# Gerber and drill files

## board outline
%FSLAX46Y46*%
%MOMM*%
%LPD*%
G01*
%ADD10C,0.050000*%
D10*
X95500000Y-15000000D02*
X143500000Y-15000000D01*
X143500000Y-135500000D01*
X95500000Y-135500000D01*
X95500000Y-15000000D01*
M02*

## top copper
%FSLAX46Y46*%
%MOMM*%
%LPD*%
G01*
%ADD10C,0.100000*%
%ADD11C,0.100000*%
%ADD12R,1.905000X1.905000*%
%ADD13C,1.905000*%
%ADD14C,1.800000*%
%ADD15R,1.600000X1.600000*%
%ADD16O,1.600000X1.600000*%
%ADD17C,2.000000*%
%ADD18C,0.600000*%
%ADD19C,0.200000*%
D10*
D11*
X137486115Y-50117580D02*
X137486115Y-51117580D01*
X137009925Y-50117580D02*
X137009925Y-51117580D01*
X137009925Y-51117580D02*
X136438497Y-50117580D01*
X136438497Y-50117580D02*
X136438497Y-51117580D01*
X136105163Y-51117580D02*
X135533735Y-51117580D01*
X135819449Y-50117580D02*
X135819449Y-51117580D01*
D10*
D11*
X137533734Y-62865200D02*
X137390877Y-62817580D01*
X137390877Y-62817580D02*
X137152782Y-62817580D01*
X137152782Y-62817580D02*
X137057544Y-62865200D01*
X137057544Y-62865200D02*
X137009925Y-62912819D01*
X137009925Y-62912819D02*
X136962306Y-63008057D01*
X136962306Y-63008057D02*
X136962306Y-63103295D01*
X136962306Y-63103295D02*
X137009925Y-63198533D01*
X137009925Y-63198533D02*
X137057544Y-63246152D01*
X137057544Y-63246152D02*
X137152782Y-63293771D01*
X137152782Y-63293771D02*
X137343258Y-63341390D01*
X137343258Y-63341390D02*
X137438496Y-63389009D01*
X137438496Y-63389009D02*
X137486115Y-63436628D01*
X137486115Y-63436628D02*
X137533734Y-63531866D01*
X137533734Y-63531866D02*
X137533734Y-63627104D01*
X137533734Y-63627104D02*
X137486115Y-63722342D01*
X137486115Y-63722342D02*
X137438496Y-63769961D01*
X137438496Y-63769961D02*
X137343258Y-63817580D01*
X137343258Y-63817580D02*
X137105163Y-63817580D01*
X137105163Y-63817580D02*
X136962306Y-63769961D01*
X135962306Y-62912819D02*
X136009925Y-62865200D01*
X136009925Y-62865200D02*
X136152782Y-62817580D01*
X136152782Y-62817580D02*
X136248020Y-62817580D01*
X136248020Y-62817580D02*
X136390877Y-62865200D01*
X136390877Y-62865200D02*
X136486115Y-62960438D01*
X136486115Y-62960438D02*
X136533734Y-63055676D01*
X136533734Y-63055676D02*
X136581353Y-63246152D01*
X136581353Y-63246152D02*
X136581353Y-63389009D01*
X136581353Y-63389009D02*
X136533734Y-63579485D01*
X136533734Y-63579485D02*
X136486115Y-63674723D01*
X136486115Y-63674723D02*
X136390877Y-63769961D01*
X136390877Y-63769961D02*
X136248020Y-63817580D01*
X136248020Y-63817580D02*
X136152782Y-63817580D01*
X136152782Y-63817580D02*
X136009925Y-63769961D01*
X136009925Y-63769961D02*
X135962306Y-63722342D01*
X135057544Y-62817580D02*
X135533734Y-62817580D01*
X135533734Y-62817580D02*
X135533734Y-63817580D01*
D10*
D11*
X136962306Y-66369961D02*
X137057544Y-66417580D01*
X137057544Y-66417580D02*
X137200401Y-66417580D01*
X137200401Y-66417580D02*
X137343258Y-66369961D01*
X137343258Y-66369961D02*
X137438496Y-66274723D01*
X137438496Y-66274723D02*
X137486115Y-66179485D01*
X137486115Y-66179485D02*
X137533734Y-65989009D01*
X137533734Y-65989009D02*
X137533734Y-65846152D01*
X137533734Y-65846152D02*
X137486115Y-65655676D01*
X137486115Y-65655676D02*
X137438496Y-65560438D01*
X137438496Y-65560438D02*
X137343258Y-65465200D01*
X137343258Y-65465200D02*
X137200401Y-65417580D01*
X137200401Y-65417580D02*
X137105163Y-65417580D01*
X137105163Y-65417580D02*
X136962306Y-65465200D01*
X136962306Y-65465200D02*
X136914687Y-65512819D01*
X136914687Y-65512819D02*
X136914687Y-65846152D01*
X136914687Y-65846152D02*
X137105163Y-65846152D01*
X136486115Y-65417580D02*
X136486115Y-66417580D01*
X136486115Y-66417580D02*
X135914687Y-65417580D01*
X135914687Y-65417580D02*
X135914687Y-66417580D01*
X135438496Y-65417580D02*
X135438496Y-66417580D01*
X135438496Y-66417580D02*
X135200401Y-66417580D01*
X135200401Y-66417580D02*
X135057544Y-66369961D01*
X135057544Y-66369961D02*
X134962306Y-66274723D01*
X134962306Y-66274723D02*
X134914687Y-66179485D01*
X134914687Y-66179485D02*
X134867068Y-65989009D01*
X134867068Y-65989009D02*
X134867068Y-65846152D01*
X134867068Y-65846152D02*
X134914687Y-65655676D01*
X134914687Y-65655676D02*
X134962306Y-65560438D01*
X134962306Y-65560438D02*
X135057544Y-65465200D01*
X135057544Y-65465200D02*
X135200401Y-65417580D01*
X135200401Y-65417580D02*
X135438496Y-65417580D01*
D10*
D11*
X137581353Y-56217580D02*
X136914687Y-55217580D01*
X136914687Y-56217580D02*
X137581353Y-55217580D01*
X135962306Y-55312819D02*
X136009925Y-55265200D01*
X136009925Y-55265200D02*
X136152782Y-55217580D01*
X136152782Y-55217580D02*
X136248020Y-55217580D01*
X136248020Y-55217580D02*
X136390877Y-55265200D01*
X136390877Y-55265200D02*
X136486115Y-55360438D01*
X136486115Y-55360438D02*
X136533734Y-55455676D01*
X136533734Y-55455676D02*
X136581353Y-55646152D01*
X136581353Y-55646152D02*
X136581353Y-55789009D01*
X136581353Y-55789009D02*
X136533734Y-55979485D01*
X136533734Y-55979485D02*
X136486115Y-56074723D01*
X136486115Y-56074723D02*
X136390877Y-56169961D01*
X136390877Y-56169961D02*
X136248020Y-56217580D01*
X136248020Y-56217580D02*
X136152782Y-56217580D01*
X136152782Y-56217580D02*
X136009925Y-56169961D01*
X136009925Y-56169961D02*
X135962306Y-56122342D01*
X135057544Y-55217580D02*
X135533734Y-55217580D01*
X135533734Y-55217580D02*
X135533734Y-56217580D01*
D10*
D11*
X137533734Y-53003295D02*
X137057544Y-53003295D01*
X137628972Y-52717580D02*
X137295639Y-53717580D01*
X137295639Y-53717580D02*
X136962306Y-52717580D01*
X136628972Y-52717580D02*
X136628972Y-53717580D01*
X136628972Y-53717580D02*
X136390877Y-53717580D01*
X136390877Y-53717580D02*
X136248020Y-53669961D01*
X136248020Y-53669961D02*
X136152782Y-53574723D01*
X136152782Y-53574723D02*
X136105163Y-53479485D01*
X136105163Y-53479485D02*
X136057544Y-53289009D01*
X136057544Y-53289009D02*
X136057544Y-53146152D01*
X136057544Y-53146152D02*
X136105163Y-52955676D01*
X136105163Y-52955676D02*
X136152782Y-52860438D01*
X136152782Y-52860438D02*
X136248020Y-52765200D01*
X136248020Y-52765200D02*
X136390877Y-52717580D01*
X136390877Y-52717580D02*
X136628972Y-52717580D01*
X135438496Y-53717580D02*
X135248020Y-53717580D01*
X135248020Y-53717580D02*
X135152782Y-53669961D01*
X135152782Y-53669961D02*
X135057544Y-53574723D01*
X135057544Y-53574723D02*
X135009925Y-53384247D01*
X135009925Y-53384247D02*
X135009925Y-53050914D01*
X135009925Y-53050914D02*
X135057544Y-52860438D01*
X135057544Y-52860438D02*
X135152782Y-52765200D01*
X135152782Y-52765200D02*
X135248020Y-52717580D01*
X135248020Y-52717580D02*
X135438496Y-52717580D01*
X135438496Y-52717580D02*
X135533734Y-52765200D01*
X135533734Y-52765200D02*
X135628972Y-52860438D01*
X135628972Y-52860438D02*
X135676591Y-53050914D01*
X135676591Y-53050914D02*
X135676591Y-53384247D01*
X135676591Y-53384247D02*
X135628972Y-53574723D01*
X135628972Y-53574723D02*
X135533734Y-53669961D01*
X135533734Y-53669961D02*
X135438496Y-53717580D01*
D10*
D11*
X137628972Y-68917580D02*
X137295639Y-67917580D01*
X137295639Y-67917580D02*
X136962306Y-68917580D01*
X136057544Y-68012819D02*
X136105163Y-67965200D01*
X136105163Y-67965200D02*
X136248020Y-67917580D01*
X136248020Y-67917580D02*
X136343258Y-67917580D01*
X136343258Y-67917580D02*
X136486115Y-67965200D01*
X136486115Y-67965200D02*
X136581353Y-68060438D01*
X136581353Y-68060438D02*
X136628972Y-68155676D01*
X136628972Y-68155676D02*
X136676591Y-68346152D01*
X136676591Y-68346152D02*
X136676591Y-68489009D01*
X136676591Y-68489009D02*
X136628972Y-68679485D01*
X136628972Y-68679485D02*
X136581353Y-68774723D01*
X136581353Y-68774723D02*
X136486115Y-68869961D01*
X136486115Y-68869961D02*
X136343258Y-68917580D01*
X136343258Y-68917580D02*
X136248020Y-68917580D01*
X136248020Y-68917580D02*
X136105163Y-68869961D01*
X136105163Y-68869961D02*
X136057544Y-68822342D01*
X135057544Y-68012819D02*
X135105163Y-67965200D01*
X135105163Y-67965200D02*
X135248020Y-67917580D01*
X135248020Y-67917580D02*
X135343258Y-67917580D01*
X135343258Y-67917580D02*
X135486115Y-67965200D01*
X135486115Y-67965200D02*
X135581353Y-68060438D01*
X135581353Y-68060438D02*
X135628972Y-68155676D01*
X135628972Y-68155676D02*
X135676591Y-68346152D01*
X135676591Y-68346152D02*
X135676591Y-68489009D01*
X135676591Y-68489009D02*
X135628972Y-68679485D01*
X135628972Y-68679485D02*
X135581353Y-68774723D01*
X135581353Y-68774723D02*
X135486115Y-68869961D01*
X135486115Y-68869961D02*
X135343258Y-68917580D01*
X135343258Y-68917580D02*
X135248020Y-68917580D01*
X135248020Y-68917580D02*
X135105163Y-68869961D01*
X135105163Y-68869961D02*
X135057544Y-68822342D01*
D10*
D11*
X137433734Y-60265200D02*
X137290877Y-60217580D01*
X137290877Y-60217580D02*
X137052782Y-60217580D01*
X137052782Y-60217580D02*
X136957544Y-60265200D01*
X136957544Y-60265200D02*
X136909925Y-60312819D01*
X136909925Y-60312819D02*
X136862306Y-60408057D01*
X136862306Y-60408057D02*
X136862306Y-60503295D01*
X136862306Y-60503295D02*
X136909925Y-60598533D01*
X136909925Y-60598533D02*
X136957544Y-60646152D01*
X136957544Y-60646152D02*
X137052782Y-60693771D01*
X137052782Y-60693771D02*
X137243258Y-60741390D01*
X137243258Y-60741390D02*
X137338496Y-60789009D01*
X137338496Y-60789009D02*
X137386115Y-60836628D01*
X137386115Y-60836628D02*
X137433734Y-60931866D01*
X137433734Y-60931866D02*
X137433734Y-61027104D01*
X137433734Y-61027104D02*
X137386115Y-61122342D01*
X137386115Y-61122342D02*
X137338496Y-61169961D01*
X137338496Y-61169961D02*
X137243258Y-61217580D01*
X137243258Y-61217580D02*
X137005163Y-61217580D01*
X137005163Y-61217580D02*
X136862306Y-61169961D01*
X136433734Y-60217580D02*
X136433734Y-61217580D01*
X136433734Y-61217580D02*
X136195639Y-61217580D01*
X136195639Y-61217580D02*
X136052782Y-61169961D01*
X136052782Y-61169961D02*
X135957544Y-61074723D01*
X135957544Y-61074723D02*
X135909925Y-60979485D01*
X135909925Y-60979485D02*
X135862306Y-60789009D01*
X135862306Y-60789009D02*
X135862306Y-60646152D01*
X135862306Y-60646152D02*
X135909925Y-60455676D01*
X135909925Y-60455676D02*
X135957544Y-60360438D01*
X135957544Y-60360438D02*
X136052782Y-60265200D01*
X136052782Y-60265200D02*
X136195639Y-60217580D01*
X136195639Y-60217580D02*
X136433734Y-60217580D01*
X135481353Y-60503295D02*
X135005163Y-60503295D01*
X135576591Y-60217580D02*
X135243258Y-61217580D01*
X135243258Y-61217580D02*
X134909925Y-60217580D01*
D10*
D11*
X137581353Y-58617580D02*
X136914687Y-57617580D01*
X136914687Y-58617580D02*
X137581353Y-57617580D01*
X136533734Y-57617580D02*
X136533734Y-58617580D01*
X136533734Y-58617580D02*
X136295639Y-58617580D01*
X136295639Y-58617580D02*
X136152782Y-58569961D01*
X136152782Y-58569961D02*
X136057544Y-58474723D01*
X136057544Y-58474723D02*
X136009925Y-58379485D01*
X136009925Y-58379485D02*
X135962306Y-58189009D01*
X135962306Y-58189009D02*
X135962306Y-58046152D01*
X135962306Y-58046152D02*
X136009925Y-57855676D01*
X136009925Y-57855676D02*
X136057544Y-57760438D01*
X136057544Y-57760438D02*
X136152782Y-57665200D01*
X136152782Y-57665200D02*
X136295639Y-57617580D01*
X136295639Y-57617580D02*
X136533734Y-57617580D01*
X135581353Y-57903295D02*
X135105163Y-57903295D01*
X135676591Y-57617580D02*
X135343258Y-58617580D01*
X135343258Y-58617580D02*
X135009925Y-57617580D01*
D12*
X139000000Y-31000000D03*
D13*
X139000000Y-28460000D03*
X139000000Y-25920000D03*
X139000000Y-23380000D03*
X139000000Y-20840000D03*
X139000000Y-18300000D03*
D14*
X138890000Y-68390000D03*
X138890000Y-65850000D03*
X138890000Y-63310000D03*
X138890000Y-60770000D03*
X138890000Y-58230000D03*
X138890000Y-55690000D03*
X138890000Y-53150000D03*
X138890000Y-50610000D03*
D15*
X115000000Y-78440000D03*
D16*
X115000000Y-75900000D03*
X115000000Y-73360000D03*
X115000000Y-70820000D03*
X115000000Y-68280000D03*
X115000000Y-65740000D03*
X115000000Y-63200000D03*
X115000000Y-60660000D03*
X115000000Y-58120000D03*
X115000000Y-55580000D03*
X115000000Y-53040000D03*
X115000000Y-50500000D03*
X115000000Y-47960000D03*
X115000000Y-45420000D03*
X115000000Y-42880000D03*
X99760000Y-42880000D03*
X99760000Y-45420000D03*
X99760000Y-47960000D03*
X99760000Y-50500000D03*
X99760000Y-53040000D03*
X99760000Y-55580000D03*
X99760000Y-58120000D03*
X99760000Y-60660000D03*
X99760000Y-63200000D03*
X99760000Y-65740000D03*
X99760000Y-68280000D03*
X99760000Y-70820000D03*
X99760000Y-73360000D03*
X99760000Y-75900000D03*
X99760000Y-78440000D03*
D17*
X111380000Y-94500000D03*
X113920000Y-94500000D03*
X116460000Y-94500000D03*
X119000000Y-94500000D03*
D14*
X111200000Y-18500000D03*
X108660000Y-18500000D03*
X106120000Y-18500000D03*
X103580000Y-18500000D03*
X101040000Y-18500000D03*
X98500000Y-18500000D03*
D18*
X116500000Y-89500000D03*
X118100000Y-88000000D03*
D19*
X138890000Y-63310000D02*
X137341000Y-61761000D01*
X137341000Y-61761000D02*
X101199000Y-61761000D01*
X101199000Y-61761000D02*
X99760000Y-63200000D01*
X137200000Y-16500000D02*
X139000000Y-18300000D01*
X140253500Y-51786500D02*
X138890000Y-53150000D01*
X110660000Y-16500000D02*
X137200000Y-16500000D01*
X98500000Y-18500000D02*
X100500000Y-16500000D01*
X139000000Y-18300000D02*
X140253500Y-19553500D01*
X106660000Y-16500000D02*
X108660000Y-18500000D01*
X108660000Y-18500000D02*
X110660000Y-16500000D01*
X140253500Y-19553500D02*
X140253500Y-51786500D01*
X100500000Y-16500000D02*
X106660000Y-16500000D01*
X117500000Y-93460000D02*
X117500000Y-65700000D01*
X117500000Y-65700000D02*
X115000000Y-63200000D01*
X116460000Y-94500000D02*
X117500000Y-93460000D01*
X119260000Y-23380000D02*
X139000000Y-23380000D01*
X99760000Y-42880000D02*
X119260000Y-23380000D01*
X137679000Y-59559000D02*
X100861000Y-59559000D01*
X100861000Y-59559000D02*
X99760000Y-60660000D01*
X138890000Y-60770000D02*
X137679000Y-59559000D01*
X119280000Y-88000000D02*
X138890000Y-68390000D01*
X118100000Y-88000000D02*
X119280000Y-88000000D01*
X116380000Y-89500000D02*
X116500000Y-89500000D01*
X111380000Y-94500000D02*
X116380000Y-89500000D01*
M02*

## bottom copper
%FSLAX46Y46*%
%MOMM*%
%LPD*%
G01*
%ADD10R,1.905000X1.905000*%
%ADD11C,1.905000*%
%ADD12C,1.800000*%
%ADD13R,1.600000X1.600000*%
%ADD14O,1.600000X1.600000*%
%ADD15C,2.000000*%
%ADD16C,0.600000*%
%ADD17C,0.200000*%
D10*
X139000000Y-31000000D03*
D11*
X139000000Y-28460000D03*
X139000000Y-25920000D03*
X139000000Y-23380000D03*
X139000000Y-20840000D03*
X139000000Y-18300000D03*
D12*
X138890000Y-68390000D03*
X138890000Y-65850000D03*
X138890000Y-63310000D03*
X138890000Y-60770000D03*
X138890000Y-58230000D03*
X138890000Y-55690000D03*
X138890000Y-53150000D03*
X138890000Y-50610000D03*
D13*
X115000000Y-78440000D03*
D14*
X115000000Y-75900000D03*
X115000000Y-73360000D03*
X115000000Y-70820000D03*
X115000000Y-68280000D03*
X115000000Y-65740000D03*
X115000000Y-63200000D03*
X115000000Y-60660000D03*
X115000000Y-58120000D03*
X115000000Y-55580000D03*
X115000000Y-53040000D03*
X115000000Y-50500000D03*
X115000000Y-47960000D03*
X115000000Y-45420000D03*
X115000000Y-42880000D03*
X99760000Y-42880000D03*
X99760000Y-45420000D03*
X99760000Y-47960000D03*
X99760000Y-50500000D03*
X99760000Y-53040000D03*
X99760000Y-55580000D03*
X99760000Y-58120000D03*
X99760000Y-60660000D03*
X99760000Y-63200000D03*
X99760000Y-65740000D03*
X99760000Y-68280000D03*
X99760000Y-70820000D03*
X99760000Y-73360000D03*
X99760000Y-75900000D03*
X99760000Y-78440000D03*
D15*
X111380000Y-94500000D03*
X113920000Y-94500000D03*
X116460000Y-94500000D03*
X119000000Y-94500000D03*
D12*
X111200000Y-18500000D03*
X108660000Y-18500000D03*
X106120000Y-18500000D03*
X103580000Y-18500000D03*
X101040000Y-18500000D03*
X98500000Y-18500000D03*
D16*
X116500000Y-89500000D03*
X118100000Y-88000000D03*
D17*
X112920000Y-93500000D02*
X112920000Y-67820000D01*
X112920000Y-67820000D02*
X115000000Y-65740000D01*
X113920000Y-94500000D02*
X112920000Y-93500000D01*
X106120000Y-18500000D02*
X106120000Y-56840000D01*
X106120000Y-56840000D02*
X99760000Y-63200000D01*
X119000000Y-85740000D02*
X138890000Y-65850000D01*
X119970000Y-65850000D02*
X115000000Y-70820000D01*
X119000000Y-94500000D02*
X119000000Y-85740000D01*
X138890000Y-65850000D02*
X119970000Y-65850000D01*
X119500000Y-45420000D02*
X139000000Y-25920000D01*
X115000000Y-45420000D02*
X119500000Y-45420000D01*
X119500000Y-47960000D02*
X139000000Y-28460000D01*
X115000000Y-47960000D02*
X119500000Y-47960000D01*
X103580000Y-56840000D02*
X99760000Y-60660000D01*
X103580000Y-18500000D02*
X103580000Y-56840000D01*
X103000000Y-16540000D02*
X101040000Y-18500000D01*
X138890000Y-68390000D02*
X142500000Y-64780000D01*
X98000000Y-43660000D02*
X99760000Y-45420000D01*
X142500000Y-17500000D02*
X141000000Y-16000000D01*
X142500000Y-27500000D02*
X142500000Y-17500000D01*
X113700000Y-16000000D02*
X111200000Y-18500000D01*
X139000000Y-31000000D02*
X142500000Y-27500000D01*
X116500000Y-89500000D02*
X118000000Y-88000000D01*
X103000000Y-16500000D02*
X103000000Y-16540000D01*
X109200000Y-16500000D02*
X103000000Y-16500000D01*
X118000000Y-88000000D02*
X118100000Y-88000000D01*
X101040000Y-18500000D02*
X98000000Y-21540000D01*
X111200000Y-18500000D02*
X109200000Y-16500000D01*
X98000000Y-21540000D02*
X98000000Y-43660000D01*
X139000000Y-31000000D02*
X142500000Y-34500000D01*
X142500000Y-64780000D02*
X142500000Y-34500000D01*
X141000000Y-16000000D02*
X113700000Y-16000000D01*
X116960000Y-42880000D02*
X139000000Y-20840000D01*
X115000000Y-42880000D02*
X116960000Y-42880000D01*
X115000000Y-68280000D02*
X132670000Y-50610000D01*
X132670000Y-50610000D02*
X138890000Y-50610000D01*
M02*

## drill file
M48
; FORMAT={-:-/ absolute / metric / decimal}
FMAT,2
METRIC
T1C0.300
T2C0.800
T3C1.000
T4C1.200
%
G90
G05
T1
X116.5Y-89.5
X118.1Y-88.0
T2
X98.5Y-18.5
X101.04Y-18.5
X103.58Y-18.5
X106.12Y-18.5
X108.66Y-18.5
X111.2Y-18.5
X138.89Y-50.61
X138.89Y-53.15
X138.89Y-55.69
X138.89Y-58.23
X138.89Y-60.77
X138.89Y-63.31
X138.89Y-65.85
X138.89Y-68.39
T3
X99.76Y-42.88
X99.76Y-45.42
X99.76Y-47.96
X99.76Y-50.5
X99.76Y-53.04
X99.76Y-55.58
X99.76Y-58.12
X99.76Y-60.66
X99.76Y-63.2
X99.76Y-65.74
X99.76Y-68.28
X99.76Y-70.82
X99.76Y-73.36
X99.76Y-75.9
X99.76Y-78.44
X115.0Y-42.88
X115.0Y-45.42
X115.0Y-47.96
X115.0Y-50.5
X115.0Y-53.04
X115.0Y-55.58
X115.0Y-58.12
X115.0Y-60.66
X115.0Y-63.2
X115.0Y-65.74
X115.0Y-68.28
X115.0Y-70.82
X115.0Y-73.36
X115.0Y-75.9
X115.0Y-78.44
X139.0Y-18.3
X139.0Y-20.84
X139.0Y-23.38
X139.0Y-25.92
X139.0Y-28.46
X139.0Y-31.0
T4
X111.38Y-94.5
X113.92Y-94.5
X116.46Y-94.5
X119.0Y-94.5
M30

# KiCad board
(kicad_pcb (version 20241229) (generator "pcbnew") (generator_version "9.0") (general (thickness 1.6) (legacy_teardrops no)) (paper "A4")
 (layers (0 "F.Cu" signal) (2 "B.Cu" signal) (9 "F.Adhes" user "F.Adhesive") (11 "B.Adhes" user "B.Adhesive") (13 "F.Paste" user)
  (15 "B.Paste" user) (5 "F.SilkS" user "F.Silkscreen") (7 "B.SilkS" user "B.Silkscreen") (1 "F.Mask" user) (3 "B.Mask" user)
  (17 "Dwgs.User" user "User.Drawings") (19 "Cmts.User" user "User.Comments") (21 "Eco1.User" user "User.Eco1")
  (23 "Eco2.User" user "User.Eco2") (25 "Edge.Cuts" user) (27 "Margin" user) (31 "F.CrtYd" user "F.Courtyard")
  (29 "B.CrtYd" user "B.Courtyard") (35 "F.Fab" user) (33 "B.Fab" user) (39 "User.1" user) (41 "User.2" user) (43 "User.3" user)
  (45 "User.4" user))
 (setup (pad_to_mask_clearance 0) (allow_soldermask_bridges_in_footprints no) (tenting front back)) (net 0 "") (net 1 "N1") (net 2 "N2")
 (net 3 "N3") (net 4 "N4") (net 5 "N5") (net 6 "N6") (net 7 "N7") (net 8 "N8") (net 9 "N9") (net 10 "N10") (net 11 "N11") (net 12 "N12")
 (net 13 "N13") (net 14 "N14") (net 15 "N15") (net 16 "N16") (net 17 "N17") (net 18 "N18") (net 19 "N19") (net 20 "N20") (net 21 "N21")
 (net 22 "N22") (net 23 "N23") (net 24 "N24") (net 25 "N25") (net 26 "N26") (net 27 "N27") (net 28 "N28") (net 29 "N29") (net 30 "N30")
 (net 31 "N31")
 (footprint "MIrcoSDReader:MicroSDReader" (layer "F.Cu") (at 139 31 180)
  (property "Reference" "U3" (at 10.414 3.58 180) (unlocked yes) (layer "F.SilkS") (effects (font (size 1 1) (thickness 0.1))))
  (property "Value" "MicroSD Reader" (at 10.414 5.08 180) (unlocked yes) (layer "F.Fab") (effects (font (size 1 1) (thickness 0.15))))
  (pad "1" thru_hole rect (at 0 0 180) (size 1.905 1.905) (drill 1) (layers "*.Cu" "*.Mask") (remove_unused_layers no) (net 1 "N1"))
  (pad "2" thru_hole circle (at 0 2.54 180) (size 1.905 1.905) (drill 1) (layers "*.Cu" "*.Mask") (remove_unused_layers no) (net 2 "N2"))
  (pad "3" thru_hole circle (at 0 5.08 180) (size 1.905 1.905) (drill 1) (layers "*.Cu" "*.Mask") (remove_unused_layers no) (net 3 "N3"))
  (pad "4" thru_hole circle (at 0 7.62 180) (size 1.905 1.905) (drill 1) (layers "*.Cu" "*.Mask") (remove_unused_layers no) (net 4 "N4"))
  (pad "5" thru_hole circle (at 0 10.16 180) (size 1.905 1.905) (drill 1) (layers "*.Cu" "*.Mask") (remove_unused_layers no) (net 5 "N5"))
  (pad "6" thru_hole circle (at 0 12.7 180) (size 1.905 1.905) (drill 1) (layers "*.Cu" "*.Mask") (remove_unused_layers no) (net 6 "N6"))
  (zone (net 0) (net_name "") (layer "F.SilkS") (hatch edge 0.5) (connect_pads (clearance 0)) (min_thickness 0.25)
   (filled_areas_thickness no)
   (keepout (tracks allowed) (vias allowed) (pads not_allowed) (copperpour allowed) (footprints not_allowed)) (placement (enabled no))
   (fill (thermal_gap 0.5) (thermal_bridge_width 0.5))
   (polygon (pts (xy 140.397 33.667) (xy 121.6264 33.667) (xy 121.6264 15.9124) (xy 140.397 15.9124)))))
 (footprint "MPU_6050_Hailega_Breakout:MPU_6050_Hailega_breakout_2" (layer "F.Cu") (at 138.89 68.39 180)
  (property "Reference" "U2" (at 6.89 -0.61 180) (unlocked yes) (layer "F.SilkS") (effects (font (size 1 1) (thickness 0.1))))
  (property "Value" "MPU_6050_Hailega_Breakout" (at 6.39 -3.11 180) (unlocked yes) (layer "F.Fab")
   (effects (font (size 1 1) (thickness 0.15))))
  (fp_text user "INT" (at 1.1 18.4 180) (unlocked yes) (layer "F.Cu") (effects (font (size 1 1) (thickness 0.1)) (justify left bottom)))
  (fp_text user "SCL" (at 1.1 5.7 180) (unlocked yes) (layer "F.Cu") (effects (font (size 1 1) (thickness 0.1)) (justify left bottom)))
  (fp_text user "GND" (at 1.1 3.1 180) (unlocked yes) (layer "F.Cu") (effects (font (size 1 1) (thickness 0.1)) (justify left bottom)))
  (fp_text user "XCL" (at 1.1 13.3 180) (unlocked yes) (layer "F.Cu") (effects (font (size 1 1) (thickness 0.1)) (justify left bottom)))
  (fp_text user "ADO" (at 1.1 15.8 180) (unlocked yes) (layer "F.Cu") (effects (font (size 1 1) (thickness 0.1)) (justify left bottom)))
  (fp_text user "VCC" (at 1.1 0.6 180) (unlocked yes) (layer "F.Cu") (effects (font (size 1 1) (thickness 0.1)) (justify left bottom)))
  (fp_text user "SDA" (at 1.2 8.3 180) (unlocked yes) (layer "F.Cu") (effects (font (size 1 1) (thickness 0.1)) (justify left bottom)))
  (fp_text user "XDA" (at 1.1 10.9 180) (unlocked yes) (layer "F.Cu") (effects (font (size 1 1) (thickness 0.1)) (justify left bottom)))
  (pad "1" thru_hole circle (at 0 0 180) (size 1.8 1.8) (drill 0.8) (layers "*.Cu" "*.Mask") (remove_unused_layers no) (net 1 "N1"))
  (pad "2" thru_hole circle (at 0 2.54 180) (size 1.8 1.8) (drill 0.8) (layers "*.Cu" "*.Mask") (remove_unused_layers no) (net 6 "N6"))
  (pad "3" thru_hole circle (at 0 5.08 180) (size 1.8 1.8) (drill 0.8) (layers "*.Cu" "*.Mask") (remove_unused_layers no) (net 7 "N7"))
  (pad "4" thru_hole circle (at 0 7.62 180) (size 1.8 1.8) (drill 0.8) (layers "*.Cu" "*.Mask") (remove_unused_layers no) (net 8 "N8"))
  (pad "5" thru_hole circle (at 0 10.16 180) (size 1.8 1.8) (drill 0.8) (layers "*.Cu" "*.Mask") (remove_unused_layers no) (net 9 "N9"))
  (pad "6" thru_hole circle (at 0 12.7 180) (size 1.8 1.8) (drill 0.8) (layers "*.Cu" "*.Mask") (remove_unused_layers no) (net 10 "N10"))
  (pad "7" thru_hole circle (at 0 15.24 180) (size 1.8 1.8) (drill 0.8) (layers "*.Cu" "*.Mask") (remove_unused_layers no) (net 6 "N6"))
  (pad "8" thru_hole circle (at 0 17.78 180) (size 1.8 1.8) (drill 0.8) (layers "*.Cu" "*.Mask") (remove_unused_layers no) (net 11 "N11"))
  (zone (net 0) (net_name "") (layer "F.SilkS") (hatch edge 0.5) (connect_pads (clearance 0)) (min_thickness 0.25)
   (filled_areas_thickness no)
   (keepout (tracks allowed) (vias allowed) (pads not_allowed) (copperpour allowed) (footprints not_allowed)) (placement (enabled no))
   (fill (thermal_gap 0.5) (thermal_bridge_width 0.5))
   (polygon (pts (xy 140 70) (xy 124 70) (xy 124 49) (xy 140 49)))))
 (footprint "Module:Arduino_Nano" (layer "F.Cu") (at 115 78.44 180)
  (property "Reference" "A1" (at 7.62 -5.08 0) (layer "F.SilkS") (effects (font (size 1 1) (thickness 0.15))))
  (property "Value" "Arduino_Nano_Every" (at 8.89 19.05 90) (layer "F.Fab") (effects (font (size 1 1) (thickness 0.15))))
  (pad "1" thru_hole rect (at 0 0 180) (size 1.6 1.6) (drill 1) (layers "*.Cu" "*.Mask") (remove_unused_layers no) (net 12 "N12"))
  (pad "2" thru_hole oval (at 0 2.54 180) (size 1.6 1.6) (drill 1) (layers "*.Cu" "*.Mask") (remove_unused_layers no) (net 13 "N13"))
  (pad "3" thru_hole oval (at 0 5.08 180) (size 1.6 1.6) (drill 1) (layers "*.Cu" "*.Mask") (remove_unused_layers no) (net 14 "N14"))
  (pad "4" thru_hole oval (at 0 7.62 180) (size 1.6 1.6) (drill 1) (layers "*.Cu" "*.Mask") (remove_unused_layers no) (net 6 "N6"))
  (pad "5" thru_hole oval (at 0 10.16 180) (size 1.6 1.6) (drill 1) (layers "*.Cu" "*.Mask") (remove_unused_layers no) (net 11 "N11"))
  (pad "6" thru_hole oval (at 0 12.7 180) (size 1.6 1.6) (drill 1) (layers "*.Cu" "*.Mask") (remove_unused_layers no) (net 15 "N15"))
  (pad "7" thru_hole oval (at 0 15.24 180) (size 1.6 1.6) (drill 1) (layers "*.Cu" "*.Mask") (remove_unused_layers no) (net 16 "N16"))
  (pad "8" thru_hole oval (at 0 17.78 180) (size 1.6 1.6) (drill 1) (layers "*.Cu" "*.Mask") (remove_unused_layers no) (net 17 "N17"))
  (pad "9" thru_hole oval (at 0 20.32 180) (size 1.6 1.6) (drill 1) (layers "*.Cu" "*.Mask") (remove_unused_layers no) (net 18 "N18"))
  (pad "10" thru_hole oval (at 0 22.86 180) (size 1.6 1.6) (drill 1) (layers "*.Cu" "*.Mask") (remove_unused_layers no) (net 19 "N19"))
  (pad "11" thru_hole oval (at 0 25.4 180) (size 1.6 1.6) (drill 1) (layers "*.Cu" "*.Mask") (remove_unused_layers no) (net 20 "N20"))
  (pad "12" thru_hole oval (at 0 27.94 180) (size 1.6 1.6) (drill 1) (layers "*.Cu" "*.Mask") (remove_unused_layers no) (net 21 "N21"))
  (pad "13" thru_hole oval (at 0 30.48 180) (size 1.6 1.6) (drill 1) (layers "*.Cu" "*.Mask") (remove_unused_layers no) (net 2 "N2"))
  (pad "14" thru_hole oval (at 0 33.02 180) (size 1.6 1.6) (drill 1) (layers "*.Cu" "*.Mask") (remove_unused_layers no) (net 3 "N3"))
  (pad "15" thru_hole oval (at 0 35.56 180) (size 1.6 1.6) (drill 1) (layers "*.Cu" "*.Mask") (remove_unused_layers no) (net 5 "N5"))
  (pad "16" thru_hole oval (at 15.24 35.56 180) (size 1.6 1.6) (drill 1) (layers "*.Cu" "*.Mask") (remove_unused_layers no) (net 4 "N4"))
  (pad "17" thru_hole oval (at 15.24 33.02 180) (size 1.6 1.6) (drill 1) (layers "*.Cu" "*.Mask") (remove_unused_layers no) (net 1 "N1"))
  (pad "18" thru_hole oval (at 15.24 30.48 180) (size 1.6 1.6) (drill 1) (layers "*.Cu" "*.Mask") (remove_unused_layers no) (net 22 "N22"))
  (pad "19" thru_hole oval (at 15.24 27.94 180) (size 1.6 1.6) (drill 1) (layers "*.Cu" "*.Mask") (remove_unused_layers no) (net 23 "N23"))
  (pad "20" thru_hole oval (at 15.24 25.4 180) (size 1.6 1.6) (drill 1) (layers "*.Cu" "*.Mask") (remove_unused_layers no) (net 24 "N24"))
  (pad "21" thru_hole oval (at 15.24 22.86 180) (size 1.6 1.6) (drill 1) (layers "*.Cu" "*.Mask") (remove_unused_layers no) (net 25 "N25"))
  (pad "22" thru_hole oval (at 15.24 20.32 180) (size 1.6 1.6) (drill 1) (layers "*.Cu" "*.Mask") (remove_unused_layers no) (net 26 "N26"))
  (pad "23" thru_hole oval (at 15.24 17.78 180) (size 1.6 1.6) (drill 1) (layers "*.Cu" "*.Mask") (remove_unused_layers no) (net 8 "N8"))
  (pad "24" thru_hole oval (at 15.24 15.24 180) (size 1.6 1.6) (drill 1) (layers "*.Cu" "*.Mask") (remove_unused_layers no) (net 7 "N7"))
  (pad "25" thru_hole oval (at 15.24 12.7 180) (size 1.6 1.6) (drill 1) (layers "*.Cu" "*.Mask") (remove_unused_layers no) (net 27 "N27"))
  (pad "26" thru_hole oval (at 15.24 10.16 180) (size 1.6 1.6) (drill 1) (layers "*.Cu" "*.Mask") (remove_unused_layers no) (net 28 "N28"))
  (pad "27" thru_hole oval (at 15.24 7.62 180) (size 1.6 1.6) (drill 1) (layers "*.Cu" "*.Mask") (remove_unused_layers no) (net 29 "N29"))
  (pad "28" thru_hole oval (at 15.24 5.08 180) (size 1.6 1.6) (drill 1) (layers "*.Cu" "*.Mask") (remove_unused_layers no) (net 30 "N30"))
  (pad "29" thru_hole oval (at 15.24 2.54 180) (size 1.6 1.6) (drill 1) (layers "*.Cu" "*.Mask") (remove_unused_layers no) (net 6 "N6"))
  (pad "30" thru_hole oval (at 15.24 0 180) (size 1.6 1.6) (drill 1) (layers "*.Cu" "*.Mask") (remove_unused_layers no) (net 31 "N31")))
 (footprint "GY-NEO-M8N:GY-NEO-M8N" (layer "F.Cu") (at 111.38 94.5)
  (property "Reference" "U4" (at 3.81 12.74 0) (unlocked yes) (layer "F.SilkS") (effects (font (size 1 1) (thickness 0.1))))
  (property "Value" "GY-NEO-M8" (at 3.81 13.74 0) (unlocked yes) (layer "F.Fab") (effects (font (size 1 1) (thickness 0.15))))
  (pad "1" thru_hole circle (at 0 0) (size 2 2) (drill 1.2) (layers "*.Cu" "*.Mask") (remove_unused_layers no) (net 1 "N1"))
  (pad "2" thru_hole circle (at 2.54 0) (size 2 2) (drill 1.2) (layers "*.Cu" "*.Mask") (remove_unused_layers no) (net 15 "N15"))
  (pad "3" thru_hole circle (at 5.08 0) (size 2 2) (drill 1.2) (layers "*.Cu" "*.Mask") (remove_unused_layers no) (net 16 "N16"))
  (pad "4" thru_hole circle (at 7.62 0) (size 2 2) (drill 1.2) (layers "*.Cu" "*.Mask") (remove_unused_layers no) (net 6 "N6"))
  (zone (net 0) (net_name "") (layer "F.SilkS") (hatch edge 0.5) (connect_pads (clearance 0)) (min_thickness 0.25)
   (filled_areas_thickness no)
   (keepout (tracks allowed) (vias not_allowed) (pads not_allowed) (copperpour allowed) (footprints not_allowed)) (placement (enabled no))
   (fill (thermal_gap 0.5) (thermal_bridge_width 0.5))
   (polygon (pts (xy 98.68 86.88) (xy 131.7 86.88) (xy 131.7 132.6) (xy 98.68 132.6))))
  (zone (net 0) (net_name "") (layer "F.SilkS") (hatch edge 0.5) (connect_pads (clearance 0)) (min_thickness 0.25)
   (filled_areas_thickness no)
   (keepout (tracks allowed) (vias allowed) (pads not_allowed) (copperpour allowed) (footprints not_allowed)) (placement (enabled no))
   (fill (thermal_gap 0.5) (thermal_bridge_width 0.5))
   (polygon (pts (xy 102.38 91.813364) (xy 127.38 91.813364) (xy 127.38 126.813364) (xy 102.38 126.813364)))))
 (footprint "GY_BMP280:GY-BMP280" (layer "F.Cu") (at 111.2 18.5 -90)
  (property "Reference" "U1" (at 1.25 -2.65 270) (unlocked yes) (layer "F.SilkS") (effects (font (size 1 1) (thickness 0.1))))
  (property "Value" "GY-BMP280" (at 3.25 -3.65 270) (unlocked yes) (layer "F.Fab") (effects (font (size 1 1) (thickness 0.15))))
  (pad "1" thru_hole circle (at 0 0 270) (size 1.8 1.8) (drill 0.8) (layers "*.Cu" "*.Mask") (remove_unused_layers no) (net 1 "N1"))
  (pad "2" thru_hole circle (at 0 2.54 270) (size 1.8 1.8) (drill 0.8) (layers "*.Cu" "*.Mask") (remove_unused_layers no) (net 6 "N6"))
  (pad "3" thru_hole circle (at 0 5.08 270) (size 1.8 1.8) (drill 0.8) (layers "*.Cu" "*.Mask") (remove_unused_layers no) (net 7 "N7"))
  (pad "4" thru_hole circle (at 0 7.62 270) (size 1.8 1.8) (drill 0.8) (layers "*.Cu" "*.Mask") (remove_unused_layers no) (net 8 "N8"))
  (pad "5" thru_hole circle (at 0 10.16 270) (size 1.8 1.8) (drill 0.8) (layers "*.Cu" "*.Mask") (remove_unused_layers no) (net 1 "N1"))
  (pad "6" thru_hole circle (at 0 12.7 270) (size 1.8 1.8) (drill 0.8) (layers "*.Cu" "*.Mask") (remove_unused_layers no) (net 6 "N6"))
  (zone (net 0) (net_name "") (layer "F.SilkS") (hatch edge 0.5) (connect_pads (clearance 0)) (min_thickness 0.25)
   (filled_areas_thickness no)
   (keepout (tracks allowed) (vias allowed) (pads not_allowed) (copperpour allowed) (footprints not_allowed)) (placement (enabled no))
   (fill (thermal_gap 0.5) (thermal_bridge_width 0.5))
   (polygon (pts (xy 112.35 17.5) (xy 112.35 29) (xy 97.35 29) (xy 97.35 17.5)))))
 (gr_rect (start 95.5 15) (end 143.5 135.5) (stroke (width 0.05) (type default)) (fill no) (layer "Edge.Cuts"))
 (segment (start 112.92 93.5) (end 112.92 67.82) (width 0.2) (layer "B.Cu") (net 15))
 (segment (start 112.92 67.82) (end 115 65.74) (width 0.2) (layer "B.Cu") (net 15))
 (segment (start 113.92 94.5) (end 112.92 93.5) (width 0.2) (layer "B.Cu") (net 15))
 (segment (start 138.89 63.31) (end 137.341 61.761) (width 0.2) (layer "F.Cu") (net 7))
 (segment (start 137.341 61.761) (end 101.199 61.761) (width 0.2) (layer "F.Cu") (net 7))
 (segment (start 101.199 61.761) (end 99.76 63.2) (width 0.2) (layer "F.Cu") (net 7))
 (segment (start 106.12 18.5) (end 106.12 56.84) (width 0.2) (layer "B.Cu") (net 7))
 (segment (start 106.12 56.84) (end 99.76 63.2) (width 0.2) (layer "B.Cu") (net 7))
 (segment (start 137.2 16.5) (end 139 18.3) (width 0.2) (layer "F.Cu") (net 6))
 (segment (start 140.2535 51.7865) (end 138.89 53.15) (width 0.2) (layer "F.Cu") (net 6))
 (segment (start 110.66 16.5) (end 137.2 16.5) (width 0.2) (layer "F.Cu") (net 6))
 (segment (start 98.5 18.5) (end 100.5 16.5) (width 0.2) (layer "F.Cu") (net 6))
 (segment (start 139 18.3) (end 140.2535 19.5535) (width 0.2) (layer "F.Cu") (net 6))
 (segment (start 106.66 16.5) (end 108.66 18.5) (width 0.2) (layer "F.Cu") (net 6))
 (segment (start 108.66 18.5) (end 110.66 16.5) (width 0.2) (layer "F.Cu") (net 6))
 (segment (start 140.2535 19.5535) (end 140.2535 51.7865) (width 0.2) (layer "F.Cu") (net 6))
 (segment (start 100.5 16.5) (end 106.66 16.5) (width 0.2) (layer "F.Cu") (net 6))
 (segment (start 119 85.74) (end 138.89 65.85) (width 0.2) (layer "B.Cu") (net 6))
 (segment (start 119.97 65.85) (end 115 70.82) (width 0.2) (layer "B.Cu") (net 6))
 (segment (start 119 94.5) (end 119 85.74) (width 0.2) (layer "B.Cu") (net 6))
 (segment (start 138.89 65.85) (end 119.97 65.85) (width 0.2) (layer "B.Cu") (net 6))
 (segment (start 117.5 93.46) (end 117.5 65.7) (width 0.2) (layer "F.Cu") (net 16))
 (segment (start 117.5 65.7) (end 115 63.2) (width 0.2) (layer "F.Cu") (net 16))
 (segment (start 116.46 94.5) (end 117.5 93.46) (width 0.2) (layer "F.Cu") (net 16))
 (segment (start 119.26 23.38) (end 139 23.38) (width 0.2) (layer "F.Cu") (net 4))
 (segment (start 99.76 42.88) (end 119.26 23.38) (width 0.2) (layer "F.Cu") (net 4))
 (segment (start 119.5 45.42) (end 139 25.92) (width 0.2) (layer "B.Cu") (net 3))
 (segment (start 115 45.42) (end 119.5 45.42) (width 0.2) (layer "B.Cu") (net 3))
 (segment (start 119.5 47.96) (end 139 28.46) (width 0.2) (layer "B.Cu") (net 2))
 (segment (start 115 47.96) (end 119.5 47.96) (width 0.2) (layer "B.Cu") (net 2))
 (segment (start 137.679 59.559) (end 100.861 59.559) (width 0.2) (layer "F.Cu") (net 8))
 (segment (start 100.861 59.559) (end 99.76 60.66) (width 0.2) (layer "F.Cu") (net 8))
 (segment (start 138.89 60.77) (end 137.679 59.559) (width 0.2) (layer "F.Cu") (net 8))
 (segment (start 103.58 56.84) (end 99.76 60.66) (width 0.2) (layer "B.Cu") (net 8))
 (segment (start 103.58 18.5) (end 103.58 56.84) (width 0.2) (layer "B.Cu") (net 8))
 (segment (start 119.28 88) (end 138.89 68.39) (width 0.2) (layer "F.Cu") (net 1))
 (segment (start 118.1 88) (end 119.28 88) (width 0.2) (layer "F.Cu") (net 1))
 (segment (start 116.38 89.5) (end 116.5 89.5) (width 0.2) (layer "F.Cu") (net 1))
 (segment (start 111.38 94.5) (end 116.38 89.5) (width 0.2) (layer "F.Cu") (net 1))
 (via (at 116.5 89.5) (size 0.6) (drill 0.3) (layers "F.Cu" "B.Cu") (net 1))
 (via (at 118.1 88) (size 0.6) (drill 0.3) (layers "F.Cu" "B.Cu") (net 1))
 (segment (start 103 16.54) (end 101.04 18.5) (width 0.2) (layer "B.Cu") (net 1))
 (segment (start 138.89 68.39) (end 142.5 64.78) (width 0.2) (layer "B.Cu") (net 1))
 (segment (start 98 43.66) (end 99.76 45.42) (width 0.2) (layer "B.Cu") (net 1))
 (segment (start 142.5 17.5) (end 141 16) (width 0.2) (layer "B.Cu") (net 1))
 (segment (start 142.5 27.5) (end 142.5 17.5) (width 0.2) (layer "B.Cu") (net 1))
 (segment (start 113.7 16) (end 111.2 18.5) (width 0.2) (layer "B.Cu") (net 1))
 (segment (start 139 31) (end 142.5 27.5) (width 0.2) (layer "B.Cu") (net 1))
 (segment (start 116.5 89.5) (end 118 88) (width 0.2) (layer "B.Cu") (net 1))
 (segment (start 103 16.5) (end 103 16.54) (width 0.2) (layer "B.Cu") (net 1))
 (segment (start 109.2 16.5) (end 103 16.5) (width 0.2) (layer "B.Cu") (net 1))
 (segment (start 118 88) (end 118.1 88) (width 0.2) (layer "B.Cu") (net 1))
 (segment (start 101.04 18.5) (end 98 21.54) (width 0.2) (layer "B.Cu") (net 1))
 (segment (start 111.2 18.5) (end 109.2 16.5) (width 0.2) (layer "B.Cu") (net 1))
 (segment (start 98 21.54) (end 98 43.66) (width 0.2) (layer "B.Cu") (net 1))
 (segment (start 139 31) (end 142.5 34.5) (width 0.2) (layer "B.Cu") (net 1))
 (segment (start 142.5 64.78) (end 142.5 34.5) (width 0.2) (layer "B.Cu") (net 1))
 (segment (start 141 16) (end 113.7 16) (width 0.2) (layer "B.Cu") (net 1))
 (segment (start 116.96 42.88) (end 139 20.84) (width 0.2) (layer "B.Cu") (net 5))
 (segment (start 115 42.88) (end 116.96 42.88) (width 0.2) (layer "B.Cu") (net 5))
 (segment (start 115 68.28) (end 132.67 50.61) (width 0.2) (layer "B.Cu") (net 11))
 (segment (start 132.67 50.61) (end 138.89 50.61) (width 0.2) (layer "B.Cu") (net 11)))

